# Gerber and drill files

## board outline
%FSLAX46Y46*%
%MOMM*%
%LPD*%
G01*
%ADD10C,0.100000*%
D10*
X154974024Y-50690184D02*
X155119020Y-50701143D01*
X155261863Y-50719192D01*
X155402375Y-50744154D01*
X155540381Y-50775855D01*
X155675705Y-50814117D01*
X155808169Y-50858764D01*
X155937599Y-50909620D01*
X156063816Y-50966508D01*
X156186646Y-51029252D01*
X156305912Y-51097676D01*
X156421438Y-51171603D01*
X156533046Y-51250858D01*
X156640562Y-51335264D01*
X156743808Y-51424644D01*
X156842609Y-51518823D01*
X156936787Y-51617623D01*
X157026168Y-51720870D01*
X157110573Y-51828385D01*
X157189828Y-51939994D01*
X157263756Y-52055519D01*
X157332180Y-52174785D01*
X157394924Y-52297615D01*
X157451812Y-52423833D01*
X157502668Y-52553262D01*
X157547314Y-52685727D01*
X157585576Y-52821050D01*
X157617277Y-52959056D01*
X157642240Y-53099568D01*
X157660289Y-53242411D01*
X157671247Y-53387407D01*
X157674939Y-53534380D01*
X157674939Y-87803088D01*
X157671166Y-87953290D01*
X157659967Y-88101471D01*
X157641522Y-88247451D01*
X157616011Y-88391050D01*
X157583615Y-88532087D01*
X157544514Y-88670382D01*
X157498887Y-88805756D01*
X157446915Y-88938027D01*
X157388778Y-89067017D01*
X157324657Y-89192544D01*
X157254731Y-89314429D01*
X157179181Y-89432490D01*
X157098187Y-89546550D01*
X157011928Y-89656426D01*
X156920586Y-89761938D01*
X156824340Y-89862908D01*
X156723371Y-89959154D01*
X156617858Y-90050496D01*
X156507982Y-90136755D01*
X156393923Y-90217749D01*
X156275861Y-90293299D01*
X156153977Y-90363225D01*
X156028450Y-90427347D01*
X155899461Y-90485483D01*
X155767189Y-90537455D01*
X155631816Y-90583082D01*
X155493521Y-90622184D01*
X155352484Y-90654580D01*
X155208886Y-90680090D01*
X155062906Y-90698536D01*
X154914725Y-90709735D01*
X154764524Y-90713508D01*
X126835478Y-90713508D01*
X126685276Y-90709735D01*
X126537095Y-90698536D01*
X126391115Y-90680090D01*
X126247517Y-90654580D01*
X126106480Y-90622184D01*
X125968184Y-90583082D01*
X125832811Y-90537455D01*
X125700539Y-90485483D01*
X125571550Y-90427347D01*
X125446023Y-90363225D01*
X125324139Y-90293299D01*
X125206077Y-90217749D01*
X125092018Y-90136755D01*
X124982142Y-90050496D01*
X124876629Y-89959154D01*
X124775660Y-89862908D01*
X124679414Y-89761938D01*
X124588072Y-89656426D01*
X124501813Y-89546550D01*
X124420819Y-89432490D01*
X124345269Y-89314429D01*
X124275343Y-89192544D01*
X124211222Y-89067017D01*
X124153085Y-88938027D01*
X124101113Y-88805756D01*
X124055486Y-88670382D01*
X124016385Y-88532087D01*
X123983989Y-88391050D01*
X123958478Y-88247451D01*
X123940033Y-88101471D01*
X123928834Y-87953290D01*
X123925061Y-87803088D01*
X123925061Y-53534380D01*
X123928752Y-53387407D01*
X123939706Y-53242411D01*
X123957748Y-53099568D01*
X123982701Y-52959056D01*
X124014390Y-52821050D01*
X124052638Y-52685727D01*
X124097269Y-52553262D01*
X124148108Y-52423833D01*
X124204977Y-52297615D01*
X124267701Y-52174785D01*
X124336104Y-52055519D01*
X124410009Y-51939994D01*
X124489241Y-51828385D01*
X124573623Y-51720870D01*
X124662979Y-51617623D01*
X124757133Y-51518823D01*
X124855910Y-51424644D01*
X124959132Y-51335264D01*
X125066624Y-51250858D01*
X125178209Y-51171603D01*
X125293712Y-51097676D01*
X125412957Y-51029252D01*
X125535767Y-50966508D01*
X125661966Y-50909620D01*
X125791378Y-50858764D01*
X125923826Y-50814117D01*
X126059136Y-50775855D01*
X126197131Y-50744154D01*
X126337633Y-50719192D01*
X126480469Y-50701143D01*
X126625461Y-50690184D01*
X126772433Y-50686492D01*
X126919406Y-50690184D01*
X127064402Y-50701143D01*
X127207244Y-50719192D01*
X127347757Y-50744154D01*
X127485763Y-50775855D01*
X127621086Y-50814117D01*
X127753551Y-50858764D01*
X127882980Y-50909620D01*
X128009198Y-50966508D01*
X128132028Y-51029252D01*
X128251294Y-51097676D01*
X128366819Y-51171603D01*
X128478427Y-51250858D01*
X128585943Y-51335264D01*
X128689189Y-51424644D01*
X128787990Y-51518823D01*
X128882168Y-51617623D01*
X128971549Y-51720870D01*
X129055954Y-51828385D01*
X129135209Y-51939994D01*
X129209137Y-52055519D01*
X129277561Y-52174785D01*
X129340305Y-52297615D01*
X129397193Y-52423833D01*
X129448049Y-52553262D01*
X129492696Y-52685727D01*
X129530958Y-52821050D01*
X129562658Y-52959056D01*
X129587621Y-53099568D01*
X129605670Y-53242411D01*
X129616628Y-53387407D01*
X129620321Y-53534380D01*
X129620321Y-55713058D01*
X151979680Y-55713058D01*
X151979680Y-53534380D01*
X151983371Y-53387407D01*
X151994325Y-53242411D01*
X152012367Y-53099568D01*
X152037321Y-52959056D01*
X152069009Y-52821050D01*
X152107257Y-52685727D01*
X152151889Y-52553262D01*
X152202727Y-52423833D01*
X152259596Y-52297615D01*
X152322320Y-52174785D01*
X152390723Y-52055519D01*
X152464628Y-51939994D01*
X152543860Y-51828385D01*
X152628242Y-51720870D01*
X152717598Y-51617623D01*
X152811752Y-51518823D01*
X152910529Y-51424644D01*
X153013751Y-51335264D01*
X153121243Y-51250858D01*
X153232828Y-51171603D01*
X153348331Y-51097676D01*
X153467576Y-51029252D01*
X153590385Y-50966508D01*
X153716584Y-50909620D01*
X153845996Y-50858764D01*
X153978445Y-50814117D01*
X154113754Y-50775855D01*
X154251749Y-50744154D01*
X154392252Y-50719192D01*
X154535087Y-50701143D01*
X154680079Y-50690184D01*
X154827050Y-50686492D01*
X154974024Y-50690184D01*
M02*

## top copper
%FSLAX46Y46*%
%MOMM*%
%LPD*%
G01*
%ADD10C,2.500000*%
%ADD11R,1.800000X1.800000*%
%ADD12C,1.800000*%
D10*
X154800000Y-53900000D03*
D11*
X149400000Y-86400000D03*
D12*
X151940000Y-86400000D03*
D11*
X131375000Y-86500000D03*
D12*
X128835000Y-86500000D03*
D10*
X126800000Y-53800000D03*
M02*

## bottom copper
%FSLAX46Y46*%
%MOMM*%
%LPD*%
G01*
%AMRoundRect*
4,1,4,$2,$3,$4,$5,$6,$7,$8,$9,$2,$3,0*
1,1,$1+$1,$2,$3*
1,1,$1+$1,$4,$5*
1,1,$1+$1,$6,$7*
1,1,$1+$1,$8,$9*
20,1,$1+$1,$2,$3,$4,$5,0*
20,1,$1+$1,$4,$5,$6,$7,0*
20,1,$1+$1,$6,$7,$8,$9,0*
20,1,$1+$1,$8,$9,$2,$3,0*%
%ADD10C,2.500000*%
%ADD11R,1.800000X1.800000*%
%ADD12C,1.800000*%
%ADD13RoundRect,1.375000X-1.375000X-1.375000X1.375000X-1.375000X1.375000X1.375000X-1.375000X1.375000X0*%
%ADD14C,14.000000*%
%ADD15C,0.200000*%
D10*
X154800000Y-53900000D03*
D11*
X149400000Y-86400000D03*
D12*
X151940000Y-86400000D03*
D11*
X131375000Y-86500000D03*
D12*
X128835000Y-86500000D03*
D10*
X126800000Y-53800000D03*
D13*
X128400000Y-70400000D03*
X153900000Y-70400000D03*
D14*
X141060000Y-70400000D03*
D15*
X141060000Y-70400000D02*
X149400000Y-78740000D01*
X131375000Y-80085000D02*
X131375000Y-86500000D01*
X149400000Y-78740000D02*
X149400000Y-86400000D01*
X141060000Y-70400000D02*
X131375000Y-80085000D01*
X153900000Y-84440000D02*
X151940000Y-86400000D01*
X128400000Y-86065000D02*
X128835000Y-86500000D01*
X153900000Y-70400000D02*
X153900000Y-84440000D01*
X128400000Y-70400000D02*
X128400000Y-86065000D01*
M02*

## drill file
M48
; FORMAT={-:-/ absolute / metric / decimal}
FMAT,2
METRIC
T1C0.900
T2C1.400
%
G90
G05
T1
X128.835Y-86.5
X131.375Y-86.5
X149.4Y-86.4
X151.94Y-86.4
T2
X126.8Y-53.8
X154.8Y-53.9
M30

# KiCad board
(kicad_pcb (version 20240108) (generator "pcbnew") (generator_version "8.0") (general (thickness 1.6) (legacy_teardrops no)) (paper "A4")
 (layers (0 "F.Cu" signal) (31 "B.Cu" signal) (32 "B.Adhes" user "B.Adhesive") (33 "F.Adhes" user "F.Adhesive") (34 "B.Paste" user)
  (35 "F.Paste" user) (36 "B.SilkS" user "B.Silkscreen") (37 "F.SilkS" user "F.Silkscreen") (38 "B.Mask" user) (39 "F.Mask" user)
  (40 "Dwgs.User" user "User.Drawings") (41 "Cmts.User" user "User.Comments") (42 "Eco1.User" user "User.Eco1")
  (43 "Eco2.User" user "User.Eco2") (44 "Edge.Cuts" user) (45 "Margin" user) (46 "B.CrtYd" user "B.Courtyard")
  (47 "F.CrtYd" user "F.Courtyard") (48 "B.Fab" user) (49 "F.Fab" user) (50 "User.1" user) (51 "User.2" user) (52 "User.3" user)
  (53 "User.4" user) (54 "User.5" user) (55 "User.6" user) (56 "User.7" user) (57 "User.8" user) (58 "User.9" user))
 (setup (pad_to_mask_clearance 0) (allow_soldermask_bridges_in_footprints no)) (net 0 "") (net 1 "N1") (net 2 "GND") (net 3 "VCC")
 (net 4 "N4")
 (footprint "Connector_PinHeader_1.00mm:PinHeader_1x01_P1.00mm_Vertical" (layer "F.Cu") (at 154.8 53.9)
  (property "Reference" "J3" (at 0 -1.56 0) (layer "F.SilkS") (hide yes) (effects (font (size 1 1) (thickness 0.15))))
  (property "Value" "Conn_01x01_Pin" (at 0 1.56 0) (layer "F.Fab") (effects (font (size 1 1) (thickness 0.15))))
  (pad "1" thru_hole circle (at 0 0) (size 2.5 2.5) (drill 1.4) (layers "*.Cu" "*.Mask") (remove_unused_layers no) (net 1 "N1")))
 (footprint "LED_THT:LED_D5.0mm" (layer "F.Cu") (at 149.4 86.4)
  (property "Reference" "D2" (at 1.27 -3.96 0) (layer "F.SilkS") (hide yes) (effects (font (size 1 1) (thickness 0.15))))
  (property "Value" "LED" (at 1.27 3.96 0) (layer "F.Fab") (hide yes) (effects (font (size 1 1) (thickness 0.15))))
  (pad "1" thru_hole rect (at 0 0) (size 1.8 1.8) (drill 0.9) (layers "*.Cu" "*.Mask") (remove_unused_layers no) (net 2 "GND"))
  (pad "2" thru_hole circle (at 2.54 0) (size 1.8 1.8) (drill 0.9) (layers "*.Cu" "*.Mask") (remove_unused_layers no) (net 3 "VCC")))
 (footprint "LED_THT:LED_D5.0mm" (layer "F.Cu") (at 131.375 86.5 180)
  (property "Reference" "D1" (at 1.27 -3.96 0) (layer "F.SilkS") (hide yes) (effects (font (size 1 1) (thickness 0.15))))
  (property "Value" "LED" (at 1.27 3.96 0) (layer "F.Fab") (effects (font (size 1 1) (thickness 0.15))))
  (pad "1" thru_hole rect (at 0 0 180) (size 1.8 1.8) (drill 0.9) (layers "*.Cu" "*.Mask") (remove_unused_layers no) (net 2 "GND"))
  (pad "2" thru_hole circle (at 2.54 0 180) (size 1.8 1.8) (drill 0.9) (layers "*.Cu" "*.Mask") (remove_unused_layers no) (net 3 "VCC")))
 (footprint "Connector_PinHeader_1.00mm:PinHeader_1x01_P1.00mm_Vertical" (layer "F.Cu") (at 126.8 53.8)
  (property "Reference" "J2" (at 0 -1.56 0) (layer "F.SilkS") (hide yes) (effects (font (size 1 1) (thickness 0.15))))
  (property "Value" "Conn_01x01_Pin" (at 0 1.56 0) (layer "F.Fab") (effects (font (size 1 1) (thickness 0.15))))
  (pad "1" thru_hole circle (at 0 0) (size 2.5 2.5) (drill 1.4) (layers "*.Cu" "*.Mask") (remove_unused_layers no) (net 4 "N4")))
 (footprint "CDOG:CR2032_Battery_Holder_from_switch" (layer "F.Cu") (at 141.15 70.4)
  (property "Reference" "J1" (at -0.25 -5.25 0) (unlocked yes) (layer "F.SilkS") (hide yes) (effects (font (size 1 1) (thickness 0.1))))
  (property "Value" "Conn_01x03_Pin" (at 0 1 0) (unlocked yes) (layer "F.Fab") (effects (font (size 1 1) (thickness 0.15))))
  (pad "1" smd roundrect (at -12.75 0) (size 5.5 5.5) (layers "B.Cu" "B.Paste" "B.Mask") (roundrect_rratio 0.25) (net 3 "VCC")
   (thermal_bridge_angle 45))
  (pad "2" smd roundrect (at 12.75 0) (size 5.5 5.5) (layers "B.Cu" "B.Paste" "B.Mask") (roundrect_rratio 0.25) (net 3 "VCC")
   (thermal_bridge_angle 45))
  (pad "3" smd circle (at -0.09 0) (size 14 14) (layers "B.Cu" "B.Paste" "B.Mask") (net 2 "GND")))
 (gr_poly
  (pts (xy 154.974024 50.690184) (xy 155.11902 50.701143) (xy 155.261863 50.719192) (xy 155.402375 50.744154) (xy 155.540381 50.775855)
   (xy 155.675705 50.814117) (xy 155.808169 50.858764) (xy 155.937599 50.90962) (xy 156.063816 50.966508) (xy 156.186646 51.029252)
   (xy 156.305912 51.097676) (xy 156.421438 51.171603) (xy 156.533046 51.250858) (xy 156.640562 51.335264) (xy 156.743808 51.424644)
   (xy 156.842609 51.518823) (xy 156.936787 51.617623) (xy 157.026168 51.72087) (xy 157.110573 51.828385) (xy 157.189828 51.939994)
   (xy 157.263756 52.055519) (xy 157.33218 52.174785) (xy 157.394924 52.297615) (xy 157.451812 52.423833) (xy 157.502668 52.553262)
   (xy 157.547314 52.685727) (xy 157.585576 52.82105) (xy 157.617277 52.959056) (xy 157.64224 53.099568) (xy 157.660289 53.242411)
   (xy 157.671247 53.387407) (xy 157.674939 53.53438) (xy 157.674939 87.803088) (xy 157.671166 87.95329) (xy 157.659967 88.101471)
   (xy 157.641522 88.247451) (xy 157.616011 88.39105) (xy 157.583615 88.532087) (xy 157.544514 88.670382) (xy 157.498887 88.805756)
   (xy 157.446915 88.938027) (xy 157.388778 89.067017) (xy 157.324657 89.192544) (xy 157.254731 89.314429) (xy 157.179181 89.43249)
   (xy 157.098187 89.54655) (xy 157.011928 89.656426) (xy 156.920586 89.761938) (xy 156.82434 89.862908) (xy 156.723371 89.959154)
   (xy 156.617858 90.050496) (xy 156.507982 90.136755) (xy 156.393923 90.217749) (xy 156.275861 90.293299) (xy 156.153977 90.363225)
   (xy 156.02845 90.427347) (xy 155.899461 90.485483) (xy 155.767189 90.537455) (xy 155.631816 90.583082) (xy 155.493521 90.622184)
   (xy 155.352484 90.65458) (xy 155.208886 90.68009) (xy 155.062906 90.698536) (xy 154.914725 90.709735) (xy 154.764524 90.713508)
   (xy 126.835478 90.713508) (xy 126.685276 90.709735) (xy 126.537095 90.698536) (xy 126.391115 90.68009) (xy 126.247517 90.65458)
   (xy 126.10648 90.622184) (xy 125.968184 90.583082) (xy 125.832811 90.537455) (xy 125.700539 90.485483) (xy 125.57155 90.427347)
   (xy 125.446023 90.363225) (xy 125.324139 90.293299) (xy 125.206077 90.217749) (xy 125.092018 90.136755) (xy 124.982142 90.050496)
   (xy 124.876629 89.959154) (xy 124.77566 89.862908) (xy 124.679414 89.761938) (xy 124.588072 89.656426) (xy 124.501813 89.54655)
   (xy 124.420819 89.43249) (xy 124.345269 89.314429) (xy 124.275343 89.192544) (xy 124.211222 89.067017) (xy 124.153085 88.938027)
   (xy 124.101113 88.805756) (xy 124.055486 88.670382) (xy 124.016385 88.532087) (xy 123.983989 88.39105) (xy 123.958478 88.247451)
   (xy 123.940033 88.101471) (xy 123.928834 87.95329) (xy 123.925061 87.803088) (xy 123.925061 53.53438) (xy 123.928752 53.387407)
   (xy 123.939706 53.242411) (xy 123.957748 53.099568) (xy 123.982701 52.959056) (xy 124.01439 52.82105) (xy 124.052638 52.685727)
   (xy 124.097269 52.553262) (xy 124.148108 52.423833) (xy 124.204977 52.297615) (xy 124.267701 52.174785) (xy 124.336104 52.055519)
   (xy 124.410009 51.939994) (xy 124.489241 51.828385) (xy 124.573623 51.72087) (xy 124.662979 51.617623) (xy 124.757133 51.518823)
   (xy 124.85591 51.424644) (xy 124.959132 51.335264) (xy 125.066624 51.250858) (xy 125.178209 51.171603) (xy 125.293712 51.097676)
   (xy 125.412957 51.029252) (xy 125.535767 50.966508) (xy 125.661966 50.90962) (xy 125.791378 50.858764) (xy 125.923826 50.814117)
   (xy 126.059136 50.775855) (xy 126.197131 50.744154) (xy 126.337633 50.719192) (xy 126.480469 50.701143) (xy 126.625461 50.690184)
   (xy 126.772433 50.686492) (xy 126.919406 50.690184) (xy 127.064402 50.701143) (xy 127.207244 50.719192) (xy 127.347757 50.744154)
   (xy 127.485763 50.775855) (xy 127.621086 50.814117) (xy 127.753551 50.858764) (xy 127.88298 50.90962) (xy 128.009198 50.966508)
   (xy 128.132028 51.029252) (xy 128.251294 51.097676) (xy 128.366819 51.171603) (xy 128.478427 51.250858) (xy 128.585943 51.335264)
   (xy 128.689189 51.424644) (xy 128.78799 51.518823) (xy 128.882168 51.617623) (xy 128.971549 51.72087) (xy 129.055954 51.828385)
   (xy 129.135209 51.939994) (xy 129.209137 52.055519) (xy 129.277561 52.174785) (xy 129.340305 52.297615) (xy 129.397193 52.423833)
   (xy 129.448049 52.553262) (xy 129.492696 52.685727) (xy 129.530958 52.82105) (xy 129.562658 52.959056) (xy 129.587621 53.099568)
   (xy 129.60567 53.242411) (xy 129.616628 53.387407) (xy 129.620321 53.53438) (xy 129.620321 55.713058) (xy 151.97968 55.713058)
   (xy 151.97968 53.53438) (xy 151.983371 53.387407) (xy 151.994325 53.242411) (xy 152.012367 53.099568) (xy 152.037321 52.959056)
   (xy 152.069009 52.82105) (xy 152.107257 52.685727) (xy 152.151889 52.553262) (xy 152.202727 52.423833) (xy 152.259596 52.297615)
   (xy 152.32232 52.174785) (xy 152.390723 52.055519) (xy 152.464628 51.939994) (xy 152.54386 51.828385) (xy 152.628242 51.72087)
   (xy 152.717598 51.617623) (xy 152.811752 51.518823) (xy 152.910529 51.424644) (xy 153.013751 51.335264) (xy 153.121243 51.250858)
   (xy 153.232828 51.171603) (xy 153.348331 51.097676) (xy 153.467576 51.029252) (xy 153.590385 50.966508) (xy 153.716584 50.90962)
   (xy 153.845996 50.858764) (xy 153.978445 50.814117) (xy 154.113754 50.775855) (xy 154.251749 50.744154) (xy 154.392252 50.719192)
   (xy 154.535087 50.701143) (xy 154.680079 50.690184) (xy 154.82705 50.686492))
  (stroke (width 0.1) (type solid) (color 155 141 141 1)) (fill none) (layer "Edge.Cuts"))
 (segment (start 141.06 70.4) (end 149.4 78.74) (width 0.2) (layer "B.Cu") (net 2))
 (segment (start 131.375 80.085) (end 131.375 86.5) (width 0.2) (layer "B.Cu") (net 2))
 (segment (start 149.4 78.74) (end 149.4 86.4) (width 0.2) (layer "B.Cu") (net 2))
 (segment (start 141.06 70.4) (end 131.375 80.085) (width 0.2) (layer "B.Cu") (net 2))
 (segment (start 153.9 84.44) (end 151.94 86.4) (width 0.2) (layer "B.Cu") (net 3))
 (segment (start 128.4 86.065) (end 128.835 86.5) (width 0.2) (layer "B.Cu") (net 3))
 (segment (start 153.9 70.4) (end 153.9 84.44) (width 0.2) (layer "B.Cu") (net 3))
 (segment (start 128.4 70.4) (end 128.4 86.065) (width 0.2) (layer "B.Cu") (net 3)))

